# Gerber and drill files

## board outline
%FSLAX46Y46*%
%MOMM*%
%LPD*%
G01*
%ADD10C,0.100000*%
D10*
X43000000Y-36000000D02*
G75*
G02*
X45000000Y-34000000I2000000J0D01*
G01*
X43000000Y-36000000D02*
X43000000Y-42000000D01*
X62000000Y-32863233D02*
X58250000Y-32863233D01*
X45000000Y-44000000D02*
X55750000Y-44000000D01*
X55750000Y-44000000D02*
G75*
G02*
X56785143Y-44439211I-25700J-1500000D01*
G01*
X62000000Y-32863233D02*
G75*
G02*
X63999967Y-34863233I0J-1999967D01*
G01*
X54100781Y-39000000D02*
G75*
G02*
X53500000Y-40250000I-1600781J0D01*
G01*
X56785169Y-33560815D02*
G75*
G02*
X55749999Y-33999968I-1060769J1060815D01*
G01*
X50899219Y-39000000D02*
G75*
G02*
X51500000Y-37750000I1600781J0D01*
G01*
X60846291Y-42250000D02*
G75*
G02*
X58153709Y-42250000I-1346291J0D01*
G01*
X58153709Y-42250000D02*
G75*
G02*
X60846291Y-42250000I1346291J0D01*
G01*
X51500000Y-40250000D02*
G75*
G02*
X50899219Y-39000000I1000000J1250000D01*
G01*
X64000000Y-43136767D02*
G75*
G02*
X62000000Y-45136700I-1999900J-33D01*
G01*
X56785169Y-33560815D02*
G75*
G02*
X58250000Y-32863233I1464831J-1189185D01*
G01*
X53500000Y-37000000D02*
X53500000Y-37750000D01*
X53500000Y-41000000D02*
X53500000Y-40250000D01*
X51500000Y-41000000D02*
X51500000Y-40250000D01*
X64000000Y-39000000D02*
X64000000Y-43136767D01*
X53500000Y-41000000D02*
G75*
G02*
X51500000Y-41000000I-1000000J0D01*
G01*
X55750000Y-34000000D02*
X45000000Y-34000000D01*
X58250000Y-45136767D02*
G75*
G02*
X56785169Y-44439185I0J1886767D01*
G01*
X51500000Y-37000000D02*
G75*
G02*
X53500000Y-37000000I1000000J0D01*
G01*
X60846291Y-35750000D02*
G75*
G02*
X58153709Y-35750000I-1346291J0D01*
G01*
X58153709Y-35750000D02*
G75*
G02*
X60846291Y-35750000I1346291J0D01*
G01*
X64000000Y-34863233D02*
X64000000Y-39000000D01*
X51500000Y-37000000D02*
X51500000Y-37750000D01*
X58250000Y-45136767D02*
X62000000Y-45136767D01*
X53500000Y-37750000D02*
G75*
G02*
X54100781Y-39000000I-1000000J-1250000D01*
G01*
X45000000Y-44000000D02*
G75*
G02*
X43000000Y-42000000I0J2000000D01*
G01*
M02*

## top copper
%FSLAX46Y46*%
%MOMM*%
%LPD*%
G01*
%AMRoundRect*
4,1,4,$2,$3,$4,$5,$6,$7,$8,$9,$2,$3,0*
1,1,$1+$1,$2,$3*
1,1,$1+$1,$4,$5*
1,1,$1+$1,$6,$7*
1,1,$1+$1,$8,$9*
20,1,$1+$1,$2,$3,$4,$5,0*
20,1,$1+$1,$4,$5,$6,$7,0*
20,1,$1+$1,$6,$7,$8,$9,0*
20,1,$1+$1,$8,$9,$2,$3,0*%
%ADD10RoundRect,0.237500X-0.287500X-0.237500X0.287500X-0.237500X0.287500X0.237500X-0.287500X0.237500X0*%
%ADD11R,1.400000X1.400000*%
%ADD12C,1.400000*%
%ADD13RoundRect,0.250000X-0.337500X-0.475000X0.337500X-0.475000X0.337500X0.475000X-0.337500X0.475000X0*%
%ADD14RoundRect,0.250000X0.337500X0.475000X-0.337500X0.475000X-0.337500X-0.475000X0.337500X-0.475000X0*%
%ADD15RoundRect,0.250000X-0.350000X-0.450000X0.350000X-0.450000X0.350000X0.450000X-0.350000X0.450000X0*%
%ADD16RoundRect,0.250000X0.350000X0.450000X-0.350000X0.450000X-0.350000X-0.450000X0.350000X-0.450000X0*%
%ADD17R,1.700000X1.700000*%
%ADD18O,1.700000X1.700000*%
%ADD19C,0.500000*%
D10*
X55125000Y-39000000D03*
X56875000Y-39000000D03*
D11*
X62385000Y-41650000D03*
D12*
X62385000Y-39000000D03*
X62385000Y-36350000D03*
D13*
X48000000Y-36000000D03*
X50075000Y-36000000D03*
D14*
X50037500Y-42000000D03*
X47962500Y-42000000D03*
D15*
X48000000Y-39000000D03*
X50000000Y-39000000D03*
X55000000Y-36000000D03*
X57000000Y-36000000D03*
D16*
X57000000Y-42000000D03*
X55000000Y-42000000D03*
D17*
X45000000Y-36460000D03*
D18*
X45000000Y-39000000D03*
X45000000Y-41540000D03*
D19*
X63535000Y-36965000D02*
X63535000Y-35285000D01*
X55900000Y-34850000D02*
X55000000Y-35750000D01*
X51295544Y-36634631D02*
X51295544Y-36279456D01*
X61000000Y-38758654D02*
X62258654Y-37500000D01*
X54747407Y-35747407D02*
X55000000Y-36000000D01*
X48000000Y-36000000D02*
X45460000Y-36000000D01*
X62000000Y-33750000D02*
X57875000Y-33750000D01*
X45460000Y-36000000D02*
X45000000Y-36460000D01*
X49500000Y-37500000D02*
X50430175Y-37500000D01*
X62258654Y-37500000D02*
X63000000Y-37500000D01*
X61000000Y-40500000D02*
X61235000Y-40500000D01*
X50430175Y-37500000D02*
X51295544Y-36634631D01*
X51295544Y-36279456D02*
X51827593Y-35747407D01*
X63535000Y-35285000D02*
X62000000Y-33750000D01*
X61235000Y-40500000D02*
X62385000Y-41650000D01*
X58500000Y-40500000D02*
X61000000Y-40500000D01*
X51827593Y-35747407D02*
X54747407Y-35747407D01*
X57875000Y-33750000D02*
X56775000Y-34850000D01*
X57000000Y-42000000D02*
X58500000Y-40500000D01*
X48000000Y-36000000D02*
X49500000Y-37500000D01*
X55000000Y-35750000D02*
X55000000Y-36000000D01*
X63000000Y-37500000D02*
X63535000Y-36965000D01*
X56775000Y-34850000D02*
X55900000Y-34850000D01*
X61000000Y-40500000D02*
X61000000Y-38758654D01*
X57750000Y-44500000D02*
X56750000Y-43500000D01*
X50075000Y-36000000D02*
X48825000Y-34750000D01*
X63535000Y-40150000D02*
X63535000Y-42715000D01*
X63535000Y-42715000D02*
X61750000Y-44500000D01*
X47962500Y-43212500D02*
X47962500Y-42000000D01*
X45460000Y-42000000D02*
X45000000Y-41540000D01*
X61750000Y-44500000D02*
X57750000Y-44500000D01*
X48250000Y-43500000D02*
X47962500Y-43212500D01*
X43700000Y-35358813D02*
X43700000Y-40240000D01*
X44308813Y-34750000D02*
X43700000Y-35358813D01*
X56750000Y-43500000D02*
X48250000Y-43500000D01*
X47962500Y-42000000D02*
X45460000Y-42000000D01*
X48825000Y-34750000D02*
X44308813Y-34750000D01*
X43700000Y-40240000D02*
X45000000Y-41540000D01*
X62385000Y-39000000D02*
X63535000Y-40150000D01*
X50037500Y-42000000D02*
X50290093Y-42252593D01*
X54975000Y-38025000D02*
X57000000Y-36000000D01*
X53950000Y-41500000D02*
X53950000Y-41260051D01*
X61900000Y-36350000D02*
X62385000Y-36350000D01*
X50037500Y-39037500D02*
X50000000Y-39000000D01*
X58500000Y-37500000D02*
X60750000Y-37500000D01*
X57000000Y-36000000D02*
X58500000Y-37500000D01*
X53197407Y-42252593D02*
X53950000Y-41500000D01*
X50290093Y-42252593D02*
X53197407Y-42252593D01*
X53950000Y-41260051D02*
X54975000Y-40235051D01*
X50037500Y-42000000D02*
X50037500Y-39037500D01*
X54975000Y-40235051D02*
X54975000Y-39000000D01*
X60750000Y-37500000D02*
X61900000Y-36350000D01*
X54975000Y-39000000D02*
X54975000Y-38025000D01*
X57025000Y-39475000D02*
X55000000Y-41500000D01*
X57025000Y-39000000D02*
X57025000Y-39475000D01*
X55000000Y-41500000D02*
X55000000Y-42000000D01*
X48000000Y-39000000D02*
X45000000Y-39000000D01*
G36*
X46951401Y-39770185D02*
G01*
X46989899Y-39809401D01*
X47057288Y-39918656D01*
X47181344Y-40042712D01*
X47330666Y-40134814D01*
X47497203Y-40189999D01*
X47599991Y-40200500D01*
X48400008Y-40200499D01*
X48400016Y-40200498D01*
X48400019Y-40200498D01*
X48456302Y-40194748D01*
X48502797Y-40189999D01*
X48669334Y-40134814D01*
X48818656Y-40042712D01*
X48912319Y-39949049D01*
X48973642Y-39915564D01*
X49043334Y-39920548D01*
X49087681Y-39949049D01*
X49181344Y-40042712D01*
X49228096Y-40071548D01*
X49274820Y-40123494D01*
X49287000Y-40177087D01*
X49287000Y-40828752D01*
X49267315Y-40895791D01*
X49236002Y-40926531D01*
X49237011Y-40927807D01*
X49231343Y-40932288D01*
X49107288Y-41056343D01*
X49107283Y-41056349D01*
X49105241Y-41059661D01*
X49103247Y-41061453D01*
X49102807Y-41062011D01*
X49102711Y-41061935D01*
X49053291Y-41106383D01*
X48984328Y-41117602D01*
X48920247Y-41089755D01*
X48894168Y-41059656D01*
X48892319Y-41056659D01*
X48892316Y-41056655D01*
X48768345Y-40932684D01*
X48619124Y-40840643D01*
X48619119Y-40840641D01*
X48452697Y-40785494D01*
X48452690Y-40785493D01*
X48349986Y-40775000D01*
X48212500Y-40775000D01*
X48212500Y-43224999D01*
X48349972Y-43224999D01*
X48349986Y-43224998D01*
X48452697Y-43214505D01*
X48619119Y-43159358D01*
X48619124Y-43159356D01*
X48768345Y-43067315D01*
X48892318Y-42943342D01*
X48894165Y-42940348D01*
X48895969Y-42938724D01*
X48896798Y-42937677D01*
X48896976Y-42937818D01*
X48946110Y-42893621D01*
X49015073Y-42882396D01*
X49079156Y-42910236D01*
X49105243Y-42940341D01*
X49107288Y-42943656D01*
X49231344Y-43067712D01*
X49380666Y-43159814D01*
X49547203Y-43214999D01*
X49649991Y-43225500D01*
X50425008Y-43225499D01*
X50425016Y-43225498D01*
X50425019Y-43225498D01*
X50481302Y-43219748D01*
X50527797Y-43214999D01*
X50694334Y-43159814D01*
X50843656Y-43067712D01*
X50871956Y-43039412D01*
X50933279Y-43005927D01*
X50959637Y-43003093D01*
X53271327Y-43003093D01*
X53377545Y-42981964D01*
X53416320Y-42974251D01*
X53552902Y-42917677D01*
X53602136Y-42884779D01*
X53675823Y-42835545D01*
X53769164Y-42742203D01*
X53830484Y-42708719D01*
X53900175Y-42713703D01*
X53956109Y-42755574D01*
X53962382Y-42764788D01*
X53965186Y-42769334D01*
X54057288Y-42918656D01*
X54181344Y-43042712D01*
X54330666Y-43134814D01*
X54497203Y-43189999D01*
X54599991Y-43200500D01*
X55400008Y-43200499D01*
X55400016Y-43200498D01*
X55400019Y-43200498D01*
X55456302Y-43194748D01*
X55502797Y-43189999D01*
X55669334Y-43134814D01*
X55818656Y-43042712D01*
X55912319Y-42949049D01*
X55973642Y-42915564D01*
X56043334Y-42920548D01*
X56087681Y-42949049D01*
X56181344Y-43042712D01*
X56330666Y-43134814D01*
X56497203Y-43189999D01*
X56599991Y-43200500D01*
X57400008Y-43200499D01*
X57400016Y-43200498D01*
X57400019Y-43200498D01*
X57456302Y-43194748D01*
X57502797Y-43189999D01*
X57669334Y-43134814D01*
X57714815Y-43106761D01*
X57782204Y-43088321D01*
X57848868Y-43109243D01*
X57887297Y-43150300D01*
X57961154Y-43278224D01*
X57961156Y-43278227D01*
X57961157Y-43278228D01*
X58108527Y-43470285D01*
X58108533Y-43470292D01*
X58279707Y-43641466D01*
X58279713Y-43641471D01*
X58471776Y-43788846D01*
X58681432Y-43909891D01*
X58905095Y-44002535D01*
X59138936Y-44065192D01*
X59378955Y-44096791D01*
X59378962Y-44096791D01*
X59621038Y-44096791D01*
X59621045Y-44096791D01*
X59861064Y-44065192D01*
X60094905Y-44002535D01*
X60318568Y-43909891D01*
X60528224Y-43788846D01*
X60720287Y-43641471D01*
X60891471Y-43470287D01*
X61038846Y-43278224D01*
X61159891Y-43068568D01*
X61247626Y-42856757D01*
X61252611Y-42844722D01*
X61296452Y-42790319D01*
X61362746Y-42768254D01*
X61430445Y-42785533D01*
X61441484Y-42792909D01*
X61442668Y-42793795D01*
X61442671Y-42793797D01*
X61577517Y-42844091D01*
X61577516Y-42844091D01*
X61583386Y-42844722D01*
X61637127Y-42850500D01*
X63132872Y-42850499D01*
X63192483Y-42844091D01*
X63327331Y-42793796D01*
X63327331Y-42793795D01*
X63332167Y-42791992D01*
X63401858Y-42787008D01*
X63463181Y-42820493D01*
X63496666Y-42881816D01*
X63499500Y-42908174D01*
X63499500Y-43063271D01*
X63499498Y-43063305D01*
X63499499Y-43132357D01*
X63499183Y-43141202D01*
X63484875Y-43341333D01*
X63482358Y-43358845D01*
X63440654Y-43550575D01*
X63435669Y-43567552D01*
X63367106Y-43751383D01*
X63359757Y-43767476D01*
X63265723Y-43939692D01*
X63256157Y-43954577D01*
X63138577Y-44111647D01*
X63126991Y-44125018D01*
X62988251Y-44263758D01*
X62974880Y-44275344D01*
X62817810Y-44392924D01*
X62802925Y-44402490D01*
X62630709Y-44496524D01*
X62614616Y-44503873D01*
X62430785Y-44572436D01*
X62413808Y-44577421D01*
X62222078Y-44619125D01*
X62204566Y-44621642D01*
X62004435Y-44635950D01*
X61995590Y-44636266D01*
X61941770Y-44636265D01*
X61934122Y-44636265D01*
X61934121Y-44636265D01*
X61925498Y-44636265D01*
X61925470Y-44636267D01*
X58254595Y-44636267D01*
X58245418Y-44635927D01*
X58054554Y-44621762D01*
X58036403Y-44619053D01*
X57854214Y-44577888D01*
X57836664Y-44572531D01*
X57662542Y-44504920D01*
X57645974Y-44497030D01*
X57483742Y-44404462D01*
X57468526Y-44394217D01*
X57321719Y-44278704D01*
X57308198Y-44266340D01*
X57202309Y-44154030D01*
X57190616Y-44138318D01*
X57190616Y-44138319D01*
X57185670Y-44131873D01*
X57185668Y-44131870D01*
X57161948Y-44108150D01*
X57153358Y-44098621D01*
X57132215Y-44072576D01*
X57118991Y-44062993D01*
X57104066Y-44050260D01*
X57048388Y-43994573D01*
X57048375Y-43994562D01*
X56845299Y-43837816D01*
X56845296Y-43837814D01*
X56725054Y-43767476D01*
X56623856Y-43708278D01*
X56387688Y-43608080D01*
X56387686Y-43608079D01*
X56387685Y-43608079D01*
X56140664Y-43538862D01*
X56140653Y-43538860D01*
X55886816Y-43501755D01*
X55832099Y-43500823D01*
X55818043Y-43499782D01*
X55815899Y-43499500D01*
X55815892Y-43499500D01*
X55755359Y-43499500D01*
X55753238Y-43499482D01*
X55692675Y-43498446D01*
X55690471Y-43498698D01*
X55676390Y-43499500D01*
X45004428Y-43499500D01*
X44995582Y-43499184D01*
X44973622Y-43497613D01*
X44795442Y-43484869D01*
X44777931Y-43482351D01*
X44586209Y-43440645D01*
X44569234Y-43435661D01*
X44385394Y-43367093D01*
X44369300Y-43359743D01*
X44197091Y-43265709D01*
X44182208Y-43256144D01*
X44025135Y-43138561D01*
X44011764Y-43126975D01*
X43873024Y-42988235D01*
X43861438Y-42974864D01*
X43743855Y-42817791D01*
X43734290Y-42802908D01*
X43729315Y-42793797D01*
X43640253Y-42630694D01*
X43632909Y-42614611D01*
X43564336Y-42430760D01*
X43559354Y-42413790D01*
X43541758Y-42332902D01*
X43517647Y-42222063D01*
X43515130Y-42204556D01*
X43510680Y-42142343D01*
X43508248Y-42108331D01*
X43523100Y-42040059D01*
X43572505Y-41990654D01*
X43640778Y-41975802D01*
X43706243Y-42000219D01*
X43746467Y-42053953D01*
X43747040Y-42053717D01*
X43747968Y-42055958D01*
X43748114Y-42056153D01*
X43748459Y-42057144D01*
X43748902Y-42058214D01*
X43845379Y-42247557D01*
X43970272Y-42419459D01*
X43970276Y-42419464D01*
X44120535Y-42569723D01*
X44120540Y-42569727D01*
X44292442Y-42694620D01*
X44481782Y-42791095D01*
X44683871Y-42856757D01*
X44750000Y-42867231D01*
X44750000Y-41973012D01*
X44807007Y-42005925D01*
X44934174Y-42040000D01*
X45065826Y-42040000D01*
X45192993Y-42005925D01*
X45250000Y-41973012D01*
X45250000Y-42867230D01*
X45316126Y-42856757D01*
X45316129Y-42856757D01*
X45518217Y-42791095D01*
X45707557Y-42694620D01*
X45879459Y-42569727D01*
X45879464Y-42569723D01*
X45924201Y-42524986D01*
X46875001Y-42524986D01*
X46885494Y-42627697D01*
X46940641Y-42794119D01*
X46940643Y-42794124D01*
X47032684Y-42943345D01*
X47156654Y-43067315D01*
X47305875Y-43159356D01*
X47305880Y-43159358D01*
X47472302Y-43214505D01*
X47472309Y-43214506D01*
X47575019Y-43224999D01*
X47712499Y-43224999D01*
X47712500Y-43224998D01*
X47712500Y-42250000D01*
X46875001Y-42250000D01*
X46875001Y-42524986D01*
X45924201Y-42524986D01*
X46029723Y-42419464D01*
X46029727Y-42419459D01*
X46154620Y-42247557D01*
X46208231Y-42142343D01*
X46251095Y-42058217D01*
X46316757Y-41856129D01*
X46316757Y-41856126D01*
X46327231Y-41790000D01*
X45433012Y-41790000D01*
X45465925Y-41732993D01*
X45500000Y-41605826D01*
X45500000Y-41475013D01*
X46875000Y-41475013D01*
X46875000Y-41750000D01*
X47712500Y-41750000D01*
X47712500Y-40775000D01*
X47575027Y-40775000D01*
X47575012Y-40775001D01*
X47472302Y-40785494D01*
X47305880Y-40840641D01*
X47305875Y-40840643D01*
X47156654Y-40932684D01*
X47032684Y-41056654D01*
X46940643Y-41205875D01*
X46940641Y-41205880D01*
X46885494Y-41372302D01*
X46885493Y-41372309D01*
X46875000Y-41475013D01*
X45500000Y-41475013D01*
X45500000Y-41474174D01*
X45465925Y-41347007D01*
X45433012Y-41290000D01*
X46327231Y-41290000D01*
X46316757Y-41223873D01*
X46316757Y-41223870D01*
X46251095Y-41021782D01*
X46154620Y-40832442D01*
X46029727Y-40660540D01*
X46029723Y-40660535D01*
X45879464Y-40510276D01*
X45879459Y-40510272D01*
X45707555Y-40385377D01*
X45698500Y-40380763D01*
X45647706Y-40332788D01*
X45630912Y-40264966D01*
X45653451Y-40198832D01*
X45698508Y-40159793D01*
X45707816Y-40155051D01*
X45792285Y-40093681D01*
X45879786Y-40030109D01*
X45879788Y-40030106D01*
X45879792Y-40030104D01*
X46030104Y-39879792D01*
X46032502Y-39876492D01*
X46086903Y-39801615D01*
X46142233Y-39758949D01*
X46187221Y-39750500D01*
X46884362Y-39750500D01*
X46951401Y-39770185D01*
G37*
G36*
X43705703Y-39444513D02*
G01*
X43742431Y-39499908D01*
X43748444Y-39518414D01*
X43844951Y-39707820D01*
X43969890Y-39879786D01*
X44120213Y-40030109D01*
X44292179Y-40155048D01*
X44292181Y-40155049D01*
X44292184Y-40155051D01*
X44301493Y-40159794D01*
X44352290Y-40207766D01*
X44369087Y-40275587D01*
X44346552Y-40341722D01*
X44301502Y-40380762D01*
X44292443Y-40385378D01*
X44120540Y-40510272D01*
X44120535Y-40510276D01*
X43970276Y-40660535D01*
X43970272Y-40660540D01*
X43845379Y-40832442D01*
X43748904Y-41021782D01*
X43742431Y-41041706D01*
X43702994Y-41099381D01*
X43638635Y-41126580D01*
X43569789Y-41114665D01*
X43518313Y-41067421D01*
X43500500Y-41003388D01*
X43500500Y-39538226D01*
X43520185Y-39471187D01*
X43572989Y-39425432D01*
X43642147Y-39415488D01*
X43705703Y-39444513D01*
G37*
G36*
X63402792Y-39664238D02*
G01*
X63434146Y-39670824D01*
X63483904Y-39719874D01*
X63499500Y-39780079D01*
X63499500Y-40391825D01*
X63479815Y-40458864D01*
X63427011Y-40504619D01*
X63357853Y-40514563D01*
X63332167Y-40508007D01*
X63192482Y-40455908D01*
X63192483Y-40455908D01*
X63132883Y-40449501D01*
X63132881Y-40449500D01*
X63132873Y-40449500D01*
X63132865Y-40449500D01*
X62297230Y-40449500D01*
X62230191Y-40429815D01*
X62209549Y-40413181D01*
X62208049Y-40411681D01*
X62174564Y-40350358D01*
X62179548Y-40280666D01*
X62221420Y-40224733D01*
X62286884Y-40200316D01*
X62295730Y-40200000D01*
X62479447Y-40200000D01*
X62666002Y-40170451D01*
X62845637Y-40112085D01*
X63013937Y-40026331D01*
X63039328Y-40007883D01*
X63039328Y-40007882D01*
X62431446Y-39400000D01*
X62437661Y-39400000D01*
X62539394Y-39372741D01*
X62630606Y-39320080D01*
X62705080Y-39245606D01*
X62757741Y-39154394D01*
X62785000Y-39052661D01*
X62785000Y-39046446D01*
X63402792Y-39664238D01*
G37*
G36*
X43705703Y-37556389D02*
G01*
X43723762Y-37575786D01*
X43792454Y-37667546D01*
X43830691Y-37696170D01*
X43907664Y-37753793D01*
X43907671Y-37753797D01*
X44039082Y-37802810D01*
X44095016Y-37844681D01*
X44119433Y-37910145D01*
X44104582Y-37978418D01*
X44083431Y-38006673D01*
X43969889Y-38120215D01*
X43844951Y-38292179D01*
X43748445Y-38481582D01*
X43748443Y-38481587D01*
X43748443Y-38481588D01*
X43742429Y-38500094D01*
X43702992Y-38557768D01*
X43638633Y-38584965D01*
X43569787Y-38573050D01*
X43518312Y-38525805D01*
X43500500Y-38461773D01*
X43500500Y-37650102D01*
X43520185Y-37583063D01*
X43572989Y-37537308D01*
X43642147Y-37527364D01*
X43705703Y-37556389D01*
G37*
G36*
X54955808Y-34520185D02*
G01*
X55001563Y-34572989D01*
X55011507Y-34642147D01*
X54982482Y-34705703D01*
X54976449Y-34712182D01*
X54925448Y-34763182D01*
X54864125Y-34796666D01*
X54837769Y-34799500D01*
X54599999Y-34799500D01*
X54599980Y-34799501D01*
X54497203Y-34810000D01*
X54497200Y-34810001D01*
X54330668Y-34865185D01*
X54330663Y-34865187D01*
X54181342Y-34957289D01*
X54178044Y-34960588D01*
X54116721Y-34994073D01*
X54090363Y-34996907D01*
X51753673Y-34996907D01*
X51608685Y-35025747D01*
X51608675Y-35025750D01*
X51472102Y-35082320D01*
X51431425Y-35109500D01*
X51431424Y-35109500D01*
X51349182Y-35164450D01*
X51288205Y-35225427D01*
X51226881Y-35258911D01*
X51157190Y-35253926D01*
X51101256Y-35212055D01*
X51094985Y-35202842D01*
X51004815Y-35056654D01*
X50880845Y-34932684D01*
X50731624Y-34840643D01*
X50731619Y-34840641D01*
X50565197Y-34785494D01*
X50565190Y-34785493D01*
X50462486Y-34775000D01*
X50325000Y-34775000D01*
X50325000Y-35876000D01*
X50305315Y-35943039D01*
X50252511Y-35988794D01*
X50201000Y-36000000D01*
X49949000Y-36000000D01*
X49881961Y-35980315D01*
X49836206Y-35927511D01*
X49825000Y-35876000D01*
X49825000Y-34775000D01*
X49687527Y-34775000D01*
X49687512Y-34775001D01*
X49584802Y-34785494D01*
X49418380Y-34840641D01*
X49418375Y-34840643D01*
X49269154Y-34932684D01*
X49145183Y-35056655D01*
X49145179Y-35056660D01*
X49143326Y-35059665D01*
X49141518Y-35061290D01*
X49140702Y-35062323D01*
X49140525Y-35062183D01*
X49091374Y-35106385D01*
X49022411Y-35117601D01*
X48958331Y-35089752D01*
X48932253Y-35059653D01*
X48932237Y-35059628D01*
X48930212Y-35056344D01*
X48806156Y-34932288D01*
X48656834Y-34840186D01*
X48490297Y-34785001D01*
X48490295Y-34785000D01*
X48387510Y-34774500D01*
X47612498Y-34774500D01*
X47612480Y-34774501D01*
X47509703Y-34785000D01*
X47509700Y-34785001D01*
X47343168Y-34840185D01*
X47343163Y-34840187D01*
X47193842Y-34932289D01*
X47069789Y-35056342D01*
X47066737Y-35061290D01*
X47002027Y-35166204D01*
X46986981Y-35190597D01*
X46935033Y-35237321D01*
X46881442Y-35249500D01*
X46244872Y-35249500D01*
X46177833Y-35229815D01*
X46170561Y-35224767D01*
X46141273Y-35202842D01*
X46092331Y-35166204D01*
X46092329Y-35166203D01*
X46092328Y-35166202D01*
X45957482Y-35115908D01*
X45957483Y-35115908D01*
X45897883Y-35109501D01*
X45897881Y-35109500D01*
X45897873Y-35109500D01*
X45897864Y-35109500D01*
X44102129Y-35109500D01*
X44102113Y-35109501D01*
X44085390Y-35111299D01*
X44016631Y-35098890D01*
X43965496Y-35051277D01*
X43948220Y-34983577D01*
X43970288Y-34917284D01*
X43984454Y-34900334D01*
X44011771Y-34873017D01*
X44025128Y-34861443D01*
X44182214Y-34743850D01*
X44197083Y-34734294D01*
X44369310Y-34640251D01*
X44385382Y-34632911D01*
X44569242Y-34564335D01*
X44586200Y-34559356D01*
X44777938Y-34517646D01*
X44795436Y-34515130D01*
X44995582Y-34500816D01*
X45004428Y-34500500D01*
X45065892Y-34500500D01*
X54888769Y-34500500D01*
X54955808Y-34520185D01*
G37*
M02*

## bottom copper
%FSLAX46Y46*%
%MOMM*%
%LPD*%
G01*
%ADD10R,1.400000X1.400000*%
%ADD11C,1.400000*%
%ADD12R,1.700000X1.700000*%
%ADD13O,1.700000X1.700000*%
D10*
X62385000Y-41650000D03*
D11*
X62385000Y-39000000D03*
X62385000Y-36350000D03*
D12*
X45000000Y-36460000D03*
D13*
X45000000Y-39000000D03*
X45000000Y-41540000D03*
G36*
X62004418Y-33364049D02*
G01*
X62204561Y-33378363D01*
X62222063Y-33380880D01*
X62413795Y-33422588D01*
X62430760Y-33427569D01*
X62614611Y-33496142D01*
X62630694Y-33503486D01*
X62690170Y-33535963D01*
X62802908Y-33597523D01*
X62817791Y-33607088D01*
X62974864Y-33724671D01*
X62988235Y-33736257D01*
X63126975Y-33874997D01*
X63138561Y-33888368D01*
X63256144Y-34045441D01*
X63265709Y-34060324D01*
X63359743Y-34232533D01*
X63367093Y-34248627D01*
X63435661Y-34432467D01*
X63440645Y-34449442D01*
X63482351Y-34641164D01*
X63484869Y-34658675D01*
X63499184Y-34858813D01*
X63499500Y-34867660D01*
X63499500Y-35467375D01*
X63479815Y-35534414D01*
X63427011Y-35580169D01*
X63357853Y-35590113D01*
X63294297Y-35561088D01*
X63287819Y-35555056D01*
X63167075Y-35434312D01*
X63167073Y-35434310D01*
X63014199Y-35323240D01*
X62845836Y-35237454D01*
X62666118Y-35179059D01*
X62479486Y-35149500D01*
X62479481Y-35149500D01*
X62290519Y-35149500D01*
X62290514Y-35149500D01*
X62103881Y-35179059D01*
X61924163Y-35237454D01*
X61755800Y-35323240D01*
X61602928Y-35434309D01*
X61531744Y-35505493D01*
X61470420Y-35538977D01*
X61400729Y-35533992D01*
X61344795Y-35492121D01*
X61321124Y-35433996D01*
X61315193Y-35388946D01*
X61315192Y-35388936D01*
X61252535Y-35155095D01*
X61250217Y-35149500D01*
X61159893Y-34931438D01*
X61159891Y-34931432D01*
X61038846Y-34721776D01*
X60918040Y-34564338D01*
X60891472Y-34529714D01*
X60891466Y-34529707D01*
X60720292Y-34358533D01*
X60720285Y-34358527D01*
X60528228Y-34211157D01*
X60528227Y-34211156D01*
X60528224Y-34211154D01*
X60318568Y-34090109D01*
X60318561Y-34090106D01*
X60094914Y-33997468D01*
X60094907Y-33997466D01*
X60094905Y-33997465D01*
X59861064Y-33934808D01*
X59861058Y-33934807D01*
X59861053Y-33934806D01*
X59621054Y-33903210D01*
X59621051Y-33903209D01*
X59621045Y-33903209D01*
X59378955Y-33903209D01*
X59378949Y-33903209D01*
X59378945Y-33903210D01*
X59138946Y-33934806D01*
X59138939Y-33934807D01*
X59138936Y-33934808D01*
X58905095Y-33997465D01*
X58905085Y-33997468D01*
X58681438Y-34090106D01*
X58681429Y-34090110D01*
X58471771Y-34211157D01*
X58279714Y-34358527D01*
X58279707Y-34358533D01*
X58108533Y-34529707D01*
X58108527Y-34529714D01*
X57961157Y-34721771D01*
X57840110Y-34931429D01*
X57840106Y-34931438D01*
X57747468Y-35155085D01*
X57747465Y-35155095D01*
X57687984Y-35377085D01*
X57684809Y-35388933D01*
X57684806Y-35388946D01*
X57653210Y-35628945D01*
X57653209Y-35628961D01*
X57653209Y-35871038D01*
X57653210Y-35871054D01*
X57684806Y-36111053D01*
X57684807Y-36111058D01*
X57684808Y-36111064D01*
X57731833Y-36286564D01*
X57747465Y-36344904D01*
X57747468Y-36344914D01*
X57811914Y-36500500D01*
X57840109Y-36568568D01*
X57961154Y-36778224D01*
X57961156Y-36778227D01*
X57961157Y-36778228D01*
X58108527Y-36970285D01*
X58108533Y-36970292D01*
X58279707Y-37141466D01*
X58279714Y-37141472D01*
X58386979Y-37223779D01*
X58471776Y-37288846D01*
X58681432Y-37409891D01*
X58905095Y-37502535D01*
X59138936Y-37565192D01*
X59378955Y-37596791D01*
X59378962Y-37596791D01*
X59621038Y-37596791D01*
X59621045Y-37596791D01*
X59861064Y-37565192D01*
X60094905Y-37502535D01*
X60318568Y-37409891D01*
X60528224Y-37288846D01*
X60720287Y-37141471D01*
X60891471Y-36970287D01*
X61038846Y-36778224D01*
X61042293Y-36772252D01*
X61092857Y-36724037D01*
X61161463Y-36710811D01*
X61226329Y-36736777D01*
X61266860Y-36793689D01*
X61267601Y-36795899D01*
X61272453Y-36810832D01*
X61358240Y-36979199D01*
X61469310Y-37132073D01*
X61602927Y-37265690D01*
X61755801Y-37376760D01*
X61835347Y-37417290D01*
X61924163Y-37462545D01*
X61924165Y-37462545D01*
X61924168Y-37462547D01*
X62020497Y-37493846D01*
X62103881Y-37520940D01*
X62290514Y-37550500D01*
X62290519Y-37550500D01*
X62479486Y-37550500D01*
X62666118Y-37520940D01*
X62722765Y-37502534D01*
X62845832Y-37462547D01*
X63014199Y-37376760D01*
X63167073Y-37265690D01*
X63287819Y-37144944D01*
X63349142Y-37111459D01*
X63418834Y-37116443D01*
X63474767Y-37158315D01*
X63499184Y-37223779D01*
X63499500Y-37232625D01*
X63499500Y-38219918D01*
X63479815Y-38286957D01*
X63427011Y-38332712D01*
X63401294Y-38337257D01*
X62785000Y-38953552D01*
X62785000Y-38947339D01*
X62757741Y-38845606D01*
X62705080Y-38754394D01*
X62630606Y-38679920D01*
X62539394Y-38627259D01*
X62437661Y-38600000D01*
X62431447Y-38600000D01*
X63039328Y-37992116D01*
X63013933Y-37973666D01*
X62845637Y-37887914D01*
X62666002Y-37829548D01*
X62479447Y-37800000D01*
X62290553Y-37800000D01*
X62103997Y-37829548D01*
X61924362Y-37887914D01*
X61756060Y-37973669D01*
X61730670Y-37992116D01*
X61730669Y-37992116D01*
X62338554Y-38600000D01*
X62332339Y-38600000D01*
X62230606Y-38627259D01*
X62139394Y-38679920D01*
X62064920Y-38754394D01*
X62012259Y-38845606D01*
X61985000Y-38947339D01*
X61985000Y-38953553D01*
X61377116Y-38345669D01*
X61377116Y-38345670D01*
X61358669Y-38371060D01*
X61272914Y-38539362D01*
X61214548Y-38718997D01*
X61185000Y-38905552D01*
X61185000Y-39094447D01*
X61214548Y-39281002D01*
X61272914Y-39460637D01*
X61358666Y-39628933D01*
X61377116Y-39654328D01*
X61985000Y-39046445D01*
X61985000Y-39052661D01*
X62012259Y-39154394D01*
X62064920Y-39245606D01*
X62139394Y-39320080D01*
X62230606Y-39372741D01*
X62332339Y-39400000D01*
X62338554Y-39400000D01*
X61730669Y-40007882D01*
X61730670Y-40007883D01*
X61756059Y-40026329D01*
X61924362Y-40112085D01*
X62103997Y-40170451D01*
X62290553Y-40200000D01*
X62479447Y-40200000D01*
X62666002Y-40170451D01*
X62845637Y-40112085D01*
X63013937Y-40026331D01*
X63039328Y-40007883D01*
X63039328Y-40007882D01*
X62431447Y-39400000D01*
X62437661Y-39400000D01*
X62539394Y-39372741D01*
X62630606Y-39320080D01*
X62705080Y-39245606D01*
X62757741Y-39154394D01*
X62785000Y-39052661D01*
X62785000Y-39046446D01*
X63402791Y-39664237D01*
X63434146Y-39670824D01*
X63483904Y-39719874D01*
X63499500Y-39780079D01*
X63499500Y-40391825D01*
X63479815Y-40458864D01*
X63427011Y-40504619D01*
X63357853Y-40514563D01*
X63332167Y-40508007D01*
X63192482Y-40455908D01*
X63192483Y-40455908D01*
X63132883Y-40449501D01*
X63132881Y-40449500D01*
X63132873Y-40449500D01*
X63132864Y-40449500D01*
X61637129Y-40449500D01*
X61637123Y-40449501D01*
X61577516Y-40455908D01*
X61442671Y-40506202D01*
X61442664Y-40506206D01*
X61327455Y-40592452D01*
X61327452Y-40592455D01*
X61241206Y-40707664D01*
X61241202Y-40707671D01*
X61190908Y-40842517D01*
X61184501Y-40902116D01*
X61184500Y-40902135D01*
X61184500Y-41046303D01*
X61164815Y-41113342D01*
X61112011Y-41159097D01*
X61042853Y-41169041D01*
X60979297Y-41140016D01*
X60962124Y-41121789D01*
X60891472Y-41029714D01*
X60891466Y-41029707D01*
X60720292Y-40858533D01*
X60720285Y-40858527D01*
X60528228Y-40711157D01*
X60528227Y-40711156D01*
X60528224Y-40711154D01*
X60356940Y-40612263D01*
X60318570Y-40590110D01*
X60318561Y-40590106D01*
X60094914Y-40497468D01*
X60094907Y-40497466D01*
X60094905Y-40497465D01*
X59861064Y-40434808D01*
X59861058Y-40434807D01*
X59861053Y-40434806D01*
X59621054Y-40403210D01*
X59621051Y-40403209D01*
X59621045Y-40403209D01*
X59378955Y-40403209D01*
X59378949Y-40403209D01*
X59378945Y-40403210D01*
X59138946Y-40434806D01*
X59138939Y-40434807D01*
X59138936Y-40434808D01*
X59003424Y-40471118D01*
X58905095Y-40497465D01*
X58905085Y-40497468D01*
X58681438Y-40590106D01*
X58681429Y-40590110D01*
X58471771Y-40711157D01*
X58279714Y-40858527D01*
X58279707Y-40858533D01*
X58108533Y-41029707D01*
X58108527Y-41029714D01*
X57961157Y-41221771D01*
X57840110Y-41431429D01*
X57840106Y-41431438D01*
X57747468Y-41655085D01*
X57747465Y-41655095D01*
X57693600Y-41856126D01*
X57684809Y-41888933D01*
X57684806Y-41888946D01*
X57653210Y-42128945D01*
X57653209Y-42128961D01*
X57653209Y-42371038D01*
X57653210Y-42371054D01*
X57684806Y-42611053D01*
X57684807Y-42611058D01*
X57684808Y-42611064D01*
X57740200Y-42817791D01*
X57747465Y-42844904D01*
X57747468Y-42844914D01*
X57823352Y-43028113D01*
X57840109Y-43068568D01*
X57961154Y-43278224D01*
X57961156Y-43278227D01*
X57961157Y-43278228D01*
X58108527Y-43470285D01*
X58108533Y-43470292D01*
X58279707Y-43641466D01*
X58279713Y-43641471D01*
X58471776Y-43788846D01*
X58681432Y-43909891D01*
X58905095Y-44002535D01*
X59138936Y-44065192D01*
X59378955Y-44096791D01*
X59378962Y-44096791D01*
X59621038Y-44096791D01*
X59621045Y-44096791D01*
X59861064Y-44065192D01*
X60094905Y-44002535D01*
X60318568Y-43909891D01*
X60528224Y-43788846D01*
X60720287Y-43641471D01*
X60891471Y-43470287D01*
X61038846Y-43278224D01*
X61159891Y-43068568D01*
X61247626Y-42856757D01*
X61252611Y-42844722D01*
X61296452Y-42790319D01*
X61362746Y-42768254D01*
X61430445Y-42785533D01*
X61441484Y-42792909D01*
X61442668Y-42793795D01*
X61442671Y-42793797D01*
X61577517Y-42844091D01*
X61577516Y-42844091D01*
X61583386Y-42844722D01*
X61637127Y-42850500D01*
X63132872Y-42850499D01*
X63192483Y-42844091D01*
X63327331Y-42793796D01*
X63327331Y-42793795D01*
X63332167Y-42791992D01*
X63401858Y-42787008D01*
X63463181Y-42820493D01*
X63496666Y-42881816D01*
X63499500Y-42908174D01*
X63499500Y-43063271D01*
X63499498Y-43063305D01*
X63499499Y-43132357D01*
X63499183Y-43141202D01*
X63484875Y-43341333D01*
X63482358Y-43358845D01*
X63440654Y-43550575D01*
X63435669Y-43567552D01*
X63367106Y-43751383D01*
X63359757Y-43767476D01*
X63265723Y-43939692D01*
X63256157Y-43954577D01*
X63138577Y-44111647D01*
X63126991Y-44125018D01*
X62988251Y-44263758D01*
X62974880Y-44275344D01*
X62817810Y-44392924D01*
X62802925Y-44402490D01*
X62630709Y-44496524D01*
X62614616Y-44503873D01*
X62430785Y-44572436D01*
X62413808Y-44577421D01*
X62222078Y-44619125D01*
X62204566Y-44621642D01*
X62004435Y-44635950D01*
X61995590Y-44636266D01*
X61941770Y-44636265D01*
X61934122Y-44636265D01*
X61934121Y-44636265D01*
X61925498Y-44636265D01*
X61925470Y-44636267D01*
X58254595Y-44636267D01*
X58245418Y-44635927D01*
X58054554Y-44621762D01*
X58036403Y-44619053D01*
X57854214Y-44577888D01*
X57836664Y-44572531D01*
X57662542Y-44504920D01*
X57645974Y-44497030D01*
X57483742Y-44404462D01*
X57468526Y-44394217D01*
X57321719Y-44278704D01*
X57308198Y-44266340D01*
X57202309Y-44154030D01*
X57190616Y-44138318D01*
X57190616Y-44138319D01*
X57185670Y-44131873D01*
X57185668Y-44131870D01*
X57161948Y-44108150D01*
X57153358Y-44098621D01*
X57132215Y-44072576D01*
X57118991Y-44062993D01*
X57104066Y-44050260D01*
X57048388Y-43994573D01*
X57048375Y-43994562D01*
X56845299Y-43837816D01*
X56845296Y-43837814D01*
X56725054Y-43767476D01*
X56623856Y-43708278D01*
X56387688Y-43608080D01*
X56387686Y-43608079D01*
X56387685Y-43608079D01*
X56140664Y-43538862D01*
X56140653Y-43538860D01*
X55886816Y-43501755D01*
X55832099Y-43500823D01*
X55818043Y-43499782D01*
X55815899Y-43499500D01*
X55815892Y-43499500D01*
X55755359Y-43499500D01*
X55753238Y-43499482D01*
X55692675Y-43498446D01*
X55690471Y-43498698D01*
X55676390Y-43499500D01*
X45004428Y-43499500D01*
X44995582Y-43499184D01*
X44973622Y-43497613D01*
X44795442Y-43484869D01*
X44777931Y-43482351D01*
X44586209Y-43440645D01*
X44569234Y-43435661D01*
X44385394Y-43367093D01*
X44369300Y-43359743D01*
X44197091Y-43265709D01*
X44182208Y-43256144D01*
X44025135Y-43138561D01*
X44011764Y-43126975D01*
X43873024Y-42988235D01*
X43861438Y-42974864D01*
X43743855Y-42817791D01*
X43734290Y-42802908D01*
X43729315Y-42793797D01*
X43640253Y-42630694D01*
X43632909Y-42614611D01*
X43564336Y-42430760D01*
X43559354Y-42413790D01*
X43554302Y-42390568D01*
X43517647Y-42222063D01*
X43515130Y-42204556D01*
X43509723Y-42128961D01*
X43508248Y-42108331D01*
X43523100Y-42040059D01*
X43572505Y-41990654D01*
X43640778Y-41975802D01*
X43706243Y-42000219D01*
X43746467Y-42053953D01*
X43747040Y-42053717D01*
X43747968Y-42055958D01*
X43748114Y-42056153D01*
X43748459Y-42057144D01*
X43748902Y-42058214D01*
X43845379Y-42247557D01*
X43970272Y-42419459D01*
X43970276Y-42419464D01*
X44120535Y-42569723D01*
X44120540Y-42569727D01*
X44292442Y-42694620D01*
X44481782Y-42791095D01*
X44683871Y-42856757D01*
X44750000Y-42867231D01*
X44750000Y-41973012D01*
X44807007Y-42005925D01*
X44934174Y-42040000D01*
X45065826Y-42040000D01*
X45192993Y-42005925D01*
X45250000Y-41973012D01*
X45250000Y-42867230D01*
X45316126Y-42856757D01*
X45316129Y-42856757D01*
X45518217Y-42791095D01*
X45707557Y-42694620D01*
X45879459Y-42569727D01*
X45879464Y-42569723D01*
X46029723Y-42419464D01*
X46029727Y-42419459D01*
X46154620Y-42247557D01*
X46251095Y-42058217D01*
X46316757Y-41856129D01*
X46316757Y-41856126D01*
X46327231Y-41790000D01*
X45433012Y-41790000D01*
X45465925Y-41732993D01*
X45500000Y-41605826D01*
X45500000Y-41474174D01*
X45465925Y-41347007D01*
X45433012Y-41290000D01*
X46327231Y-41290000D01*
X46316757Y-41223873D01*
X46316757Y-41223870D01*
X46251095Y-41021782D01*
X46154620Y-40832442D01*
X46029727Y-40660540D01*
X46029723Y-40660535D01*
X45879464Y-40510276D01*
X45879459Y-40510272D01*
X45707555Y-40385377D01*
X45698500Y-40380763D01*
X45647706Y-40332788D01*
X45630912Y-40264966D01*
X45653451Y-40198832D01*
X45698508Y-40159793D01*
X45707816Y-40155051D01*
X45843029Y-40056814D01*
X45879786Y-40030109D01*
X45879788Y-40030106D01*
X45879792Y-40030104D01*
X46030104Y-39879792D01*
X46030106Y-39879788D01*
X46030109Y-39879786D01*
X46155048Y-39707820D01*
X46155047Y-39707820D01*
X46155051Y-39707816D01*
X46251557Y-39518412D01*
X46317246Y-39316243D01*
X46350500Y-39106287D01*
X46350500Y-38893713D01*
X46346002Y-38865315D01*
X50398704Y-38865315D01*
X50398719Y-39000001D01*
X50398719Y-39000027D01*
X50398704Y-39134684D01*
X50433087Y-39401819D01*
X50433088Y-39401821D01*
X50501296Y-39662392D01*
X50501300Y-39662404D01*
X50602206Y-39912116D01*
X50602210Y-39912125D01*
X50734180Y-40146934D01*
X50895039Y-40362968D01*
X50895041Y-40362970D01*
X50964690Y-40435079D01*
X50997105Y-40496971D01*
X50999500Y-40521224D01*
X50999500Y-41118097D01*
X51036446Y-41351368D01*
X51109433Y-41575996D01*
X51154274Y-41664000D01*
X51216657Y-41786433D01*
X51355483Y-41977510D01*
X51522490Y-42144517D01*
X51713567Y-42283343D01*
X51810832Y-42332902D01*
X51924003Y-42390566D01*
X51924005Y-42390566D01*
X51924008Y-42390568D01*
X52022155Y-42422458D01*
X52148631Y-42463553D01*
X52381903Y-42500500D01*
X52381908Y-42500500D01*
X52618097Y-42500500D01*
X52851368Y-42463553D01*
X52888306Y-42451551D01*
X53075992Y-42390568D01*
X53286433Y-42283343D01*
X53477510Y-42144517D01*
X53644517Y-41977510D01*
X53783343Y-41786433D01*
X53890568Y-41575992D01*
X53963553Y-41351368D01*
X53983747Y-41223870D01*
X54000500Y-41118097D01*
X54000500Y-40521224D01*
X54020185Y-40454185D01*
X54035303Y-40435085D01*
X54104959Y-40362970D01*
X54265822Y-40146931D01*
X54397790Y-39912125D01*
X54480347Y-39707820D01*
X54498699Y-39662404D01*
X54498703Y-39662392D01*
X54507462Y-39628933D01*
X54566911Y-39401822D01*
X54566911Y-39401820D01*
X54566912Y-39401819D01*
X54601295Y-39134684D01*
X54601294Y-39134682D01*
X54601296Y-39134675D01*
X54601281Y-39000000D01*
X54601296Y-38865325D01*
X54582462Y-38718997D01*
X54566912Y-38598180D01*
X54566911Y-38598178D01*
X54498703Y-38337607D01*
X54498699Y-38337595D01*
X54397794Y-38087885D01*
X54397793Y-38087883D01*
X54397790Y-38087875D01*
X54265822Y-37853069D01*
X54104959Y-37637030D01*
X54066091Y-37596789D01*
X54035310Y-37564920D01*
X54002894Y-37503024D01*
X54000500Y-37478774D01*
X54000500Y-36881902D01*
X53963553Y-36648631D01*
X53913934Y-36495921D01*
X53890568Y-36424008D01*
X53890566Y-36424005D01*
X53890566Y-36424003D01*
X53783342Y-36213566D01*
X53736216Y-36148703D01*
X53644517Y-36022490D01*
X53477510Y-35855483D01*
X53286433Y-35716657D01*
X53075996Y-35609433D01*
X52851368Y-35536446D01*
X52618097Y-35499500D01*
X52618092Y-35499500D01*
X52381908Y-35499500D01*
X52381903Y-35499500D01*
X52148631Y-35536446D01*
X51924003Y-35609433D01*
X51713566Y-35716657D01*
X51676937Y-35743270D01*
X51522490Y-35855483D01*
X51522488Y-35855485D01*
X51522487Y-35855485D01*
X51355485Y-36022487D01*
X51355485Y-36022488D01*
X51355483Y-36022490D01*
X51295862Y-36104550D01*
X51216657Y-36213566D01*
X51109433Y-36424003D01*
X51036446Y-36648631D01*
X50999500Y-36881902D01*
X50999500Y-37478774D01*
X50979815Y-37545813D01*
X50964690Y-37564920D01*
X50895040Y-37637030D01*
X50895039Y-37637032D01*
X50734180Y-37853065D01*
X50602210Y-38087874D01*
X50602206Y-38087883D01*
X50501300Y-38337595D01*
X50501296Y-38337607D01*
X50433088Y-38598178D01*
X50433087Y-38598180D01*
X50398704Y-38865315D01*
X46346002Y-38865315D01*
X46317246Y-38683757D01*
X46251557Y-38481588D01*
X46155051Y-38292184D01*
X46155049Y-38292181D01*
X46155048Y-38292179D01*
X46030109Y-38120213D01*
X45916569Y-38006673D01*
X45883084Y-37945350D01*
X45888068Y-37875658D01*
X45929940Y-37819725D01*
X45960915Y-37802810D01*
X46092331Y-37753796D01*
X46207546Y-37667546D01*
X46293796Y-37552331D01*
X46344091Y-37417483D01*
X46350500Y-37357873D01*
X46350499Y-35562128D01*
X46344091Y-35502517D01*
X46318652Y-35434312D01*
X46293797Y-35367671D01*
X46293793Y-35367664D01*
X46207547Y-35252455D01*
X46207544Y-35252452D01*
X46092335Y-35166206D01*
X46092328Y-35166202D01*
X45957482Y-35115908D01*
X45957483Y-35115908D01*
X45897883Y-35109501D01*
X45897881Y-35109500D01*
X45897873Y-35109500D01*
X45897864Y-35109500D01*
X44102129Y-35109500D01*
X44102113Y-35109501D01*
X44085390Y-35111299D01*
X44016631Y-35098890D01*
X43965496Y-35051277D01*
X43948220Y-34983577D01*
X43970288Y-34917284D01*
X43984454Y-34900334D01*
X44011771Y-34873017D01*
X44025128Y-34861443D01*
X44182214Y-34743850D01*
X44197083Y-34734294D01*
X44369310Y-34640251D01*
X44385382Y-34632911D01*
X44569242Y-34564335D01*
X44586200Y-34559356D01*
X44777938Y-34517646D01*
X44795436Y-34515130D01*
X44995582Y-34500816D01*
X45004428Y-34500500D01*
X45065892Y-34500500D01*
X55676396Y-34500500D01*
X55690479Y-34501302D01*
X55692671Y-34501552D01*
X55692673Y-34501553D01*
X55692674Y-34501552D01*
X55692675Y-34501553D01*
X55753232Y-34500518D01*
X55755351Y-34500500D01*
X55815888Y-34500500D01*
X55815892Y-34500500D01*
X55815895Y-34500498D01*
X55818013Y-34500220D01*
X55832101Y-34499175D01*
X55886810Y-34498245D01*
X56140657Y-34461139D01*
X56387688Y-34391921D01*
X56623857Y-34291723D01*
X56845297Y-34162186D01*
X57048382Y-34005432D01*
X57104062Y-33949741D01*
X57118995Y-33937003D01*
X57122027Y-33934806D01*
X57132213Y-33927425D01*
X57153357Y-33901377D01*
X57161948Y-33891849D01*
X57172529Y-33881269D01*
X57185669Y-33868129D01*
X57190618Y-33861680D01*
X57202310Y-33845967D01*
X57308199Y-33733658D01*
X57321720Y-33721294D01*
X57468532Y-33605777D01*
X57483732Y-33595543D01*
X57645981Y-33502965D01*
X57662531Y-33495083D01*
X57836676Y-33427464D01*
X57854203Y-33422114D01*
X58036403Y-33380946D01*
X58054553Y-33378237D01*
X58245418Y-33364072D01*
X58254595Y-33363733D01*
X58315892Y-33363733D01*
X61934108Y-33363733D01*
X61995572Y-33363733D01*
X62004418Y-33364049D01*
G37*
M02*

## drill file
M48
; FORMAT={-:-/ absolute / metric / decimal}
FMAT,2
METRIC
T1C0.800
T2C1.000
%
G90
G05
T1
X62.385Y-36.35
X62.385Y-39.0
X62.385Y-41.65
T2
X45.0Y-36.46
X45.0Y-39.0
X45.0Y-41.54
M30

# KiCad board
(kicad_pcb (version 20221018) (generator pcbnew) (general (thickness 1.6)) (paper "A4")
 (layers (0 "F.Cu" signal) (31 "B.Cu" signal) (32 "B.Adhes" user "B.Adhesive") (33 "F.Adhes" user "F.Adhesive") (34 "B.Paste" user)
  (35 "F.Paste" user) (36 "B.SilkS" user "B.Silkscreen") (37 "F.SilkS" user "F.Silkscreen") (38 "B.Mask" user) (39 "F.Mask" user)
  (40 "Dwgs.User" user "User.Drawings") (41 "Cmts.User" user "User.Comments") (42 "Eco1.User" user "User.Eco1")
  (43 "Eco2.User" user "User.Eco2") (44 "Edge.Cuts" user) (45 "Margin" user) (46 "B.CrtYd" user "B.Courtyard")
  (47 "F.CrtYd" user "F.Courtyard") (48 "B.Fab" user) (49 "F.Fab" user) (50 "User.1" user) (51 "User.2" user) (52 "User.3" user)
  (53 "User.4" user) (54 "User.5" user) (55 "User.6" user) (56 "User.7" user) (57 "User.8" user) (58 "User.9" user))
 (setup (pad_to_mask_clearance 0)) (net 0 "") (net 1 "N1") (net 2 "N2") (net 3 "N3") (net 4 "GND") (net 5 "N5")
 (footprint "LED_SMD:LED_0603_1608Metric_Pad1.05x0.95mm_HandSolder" (layer "F.Cu") (at 56 39)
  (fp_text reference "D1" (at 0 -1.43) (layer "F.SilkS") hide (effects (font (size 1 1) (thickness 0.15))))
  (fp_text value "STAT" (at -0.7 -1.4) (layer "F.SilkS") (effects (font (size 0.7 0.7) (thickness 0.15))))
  (pad "1" smd roundrect (at -0.875 0) (size 1.05 0.95) (layers "F.Cu" "F.Paste" "F.Mask") (roundrect_rratio 0.25) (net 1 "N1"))
  (pad "2" smd roundrect (at 0.875 0) (size 1.05 0.95) (layers "F.Cu" "F.Paste" "F.Mask") (roundrect_rratio 0.25) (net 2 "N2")))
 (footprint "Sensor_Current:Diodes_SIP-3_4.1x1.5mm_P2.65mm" (layer "F.Cu") (at 62.385 41.65 90)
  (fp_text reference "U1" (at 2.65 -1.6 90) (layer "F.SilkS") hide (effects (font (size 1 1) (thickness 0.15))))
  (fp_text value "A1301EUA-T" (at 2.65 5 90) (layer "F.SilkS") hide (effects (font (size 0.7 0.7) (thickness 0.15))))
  (pad "1" thru_hole rect (at 0 0 90) (size 1.4 1.4) (drill 0.8) (layers "*.Cu" "*.Mask") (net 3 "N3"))
  (pad "2" thru_hole circle (at 2.65 0 90) (size 1.4 1.4) (drill 0.8) (layers "*.Cu" "*.Mask") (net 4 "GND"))
  (pad "3" thru_hole circle (at 5.3 0 90) (size 1.4 1.4) (drill 0.8) (layers "*.Cu" "*.Mask") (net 1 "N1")))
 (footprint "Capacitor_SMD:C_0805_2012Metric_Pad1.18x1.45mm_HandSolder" (layer "F.Cu") (at 49.0375 36)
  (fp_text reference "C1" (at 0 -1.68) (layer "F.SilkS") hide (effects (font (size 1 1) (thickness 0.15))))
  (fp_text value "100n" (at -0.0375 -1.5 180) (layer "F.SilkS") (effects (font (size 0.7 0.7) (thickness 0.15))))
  (pad "1" smd roundrect (at -1.0375 0) (size 1.175 1.45) (layers "F.Cu" "F.Paste" "F.Mask") (roundrect_rratio 0.212766) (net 3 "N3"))
  (pad "2" smd roundrect (at 1.0375 0) (size 1.175 1.45) (layers "F.Cu" "F.Paste" "F.Mask") (roundrect_rratio 0.212766) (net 4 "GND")))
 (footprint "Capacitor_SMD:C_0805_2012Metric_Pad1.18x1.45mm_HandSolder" (layer "F.Cu") (at 49 42 180)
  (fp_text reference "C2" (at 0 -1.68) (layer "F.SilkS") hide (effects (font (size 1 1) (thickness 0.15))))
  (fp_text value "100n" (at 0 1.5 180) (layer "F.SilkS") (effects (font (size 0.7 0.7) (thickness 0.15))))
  (pad "1" smd roundrect (at -1.0375 0 180) (size 1.175 1.45) (layers "F.Cu" "F.Paste" "F.Mask") (roundrect_rratio 0.212766) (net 1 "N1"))
  (pad "2" smd roundrect (at 1.0375 0 180) (size 1.175 1.45) (layers "F.Cu" "F.Paste" "F.Mask") (roundrect_rratio 0.212766) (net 4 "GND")))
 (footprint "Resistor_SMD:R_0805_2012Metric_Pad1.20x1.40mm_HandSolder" (layer "F.Cu") (at 49 39)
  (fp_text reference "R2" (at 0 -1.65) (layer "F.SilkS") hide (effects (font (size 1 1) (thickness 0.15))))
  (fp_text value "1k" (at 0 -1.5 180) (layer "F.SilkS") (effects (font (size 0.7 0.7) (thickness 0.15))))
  (pad "1" smd roundrect (at -1 0) (size 1.2 1.4) (layers "F.Cu" "F.Paste" "F.Mask") (roundrect_rratio 0.208333) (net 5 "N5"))
  (pad "2" smd roundrect (at 1 0) (size 1.2 1.4) (layers "F.Cu" "F.Paste" "F.Mask") (roundrect_rratio 0.208333) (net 1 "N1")))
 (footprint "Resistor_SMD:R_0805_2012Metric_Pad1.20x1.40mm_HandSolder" (layer "F.Cu") (at 56 36)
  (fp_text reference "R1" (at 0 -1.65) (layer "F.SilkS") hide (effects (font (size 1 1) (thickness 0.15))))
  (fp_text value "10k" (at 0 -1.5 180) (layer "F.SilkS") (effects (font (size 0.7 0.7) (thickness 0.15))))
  (pad "1" smd roundrect (at -1 0) (size 1.2 1.4) (layers "F.Cu" "F.Paste" "F.Mask") (roundrect_rratio 0.208333) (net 3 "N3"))
  (pad "2" smd roundrect (at 1 0) (size 1.2 1.4) (layers "F.Cu" "F.Paste" "F.Mask") (roundrect_rratio 0.208333) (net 1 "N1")))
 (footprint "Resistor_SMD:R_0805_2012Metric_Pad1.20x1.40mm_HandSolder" (layer "F.Cu") (at 56 42 180)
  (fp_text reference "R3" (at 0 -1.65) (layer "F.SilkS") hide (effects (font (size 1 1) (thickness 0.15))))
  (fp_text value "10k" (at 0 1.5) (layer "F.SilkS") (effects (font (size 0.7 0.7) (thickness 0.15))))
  (pad "1" smd roundrect (at -1 0 180) (size 1.2 1.4) (layers "F.Cu" "F.Paste" "F.Mask") (roundrect_rratio 0.208333) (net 3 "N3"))
  (pad "2" smd roundrect (at 1 0 180) (size 1.2 1.4) (layers "F.Cu" "F.Paste" "F.Mask") (roundrect_rratio 0.208333) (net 2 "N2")))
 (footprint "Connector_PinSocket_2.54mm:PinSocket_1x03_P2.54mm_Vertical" (layer "F.Cu") (at 45 36.46)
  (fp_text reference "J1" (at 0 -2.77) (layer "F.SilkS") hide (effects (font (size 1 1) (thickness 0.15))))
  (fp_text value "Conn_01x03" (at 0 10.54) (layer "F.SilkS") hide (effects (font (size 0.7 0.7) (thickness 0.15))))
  (pad "1" thru_hole rect (at 0 0) (size 1.7 1.7) (drill 1) (layers "*.Cu" "*.Mask") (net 3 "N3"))
  (pad "2" thru_hole oval (at 0 2.54) (size 1.7 1.7) (drill 1) (layers "*.Cu" "*.Mask") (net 5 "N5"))
  (pad "3" thru_hole oval (at 0 5.08) (size 1.7 1.7) (drill 1) (layers "*.Cu" "*.Mask") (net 4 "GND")))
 (gr_arc (start 43 36) (mid 43.585786 34.585786) (end 45 34) (stroke (width 0.1) (type default)) (layer "Edge.Cuts"))
 (gr_line (start 43 36) (end 43 42) (stroke (width 0.1) (type default)) (layer "Edge.Cuts"))
 (gr_line (start 62 32.863233) (end 58.25 32.863233) (stroke (width 0.1) (type default)) (layer "Edge.Cuts"))
 (gr_line (start 45 44) (end 55.75 44) (stroke (width 0.1) (type default)) (layer "Edge.Cuts"))
 (gr_arc (start 55.75 44) (mid 56.310289 44.118937) (end 56.785169 44.439185) (stroke (width 0.1) (type default)) (layer "Edge.Cuts"))
 (gr_arc (start 62 32.863233) (mid 63.414214 33.449019) (end 64 34.863233) (stroke (width 0.1) (type default)) (layer "Edge.Cuts"))
 (gr_arc (start 54.100781 39) (mid 53.942789 39.69344) (end 53.5 40.25) (stroke (width 0.1) (type default)) (layer "Edge.Cuts"))
 (gr_arc (start 56.785169 33.560815) (mid 56.310289 33.881064) (end 55.75 34) (stroke (width 0.1) (type default)) (layer "Edge.Cuts"))
 (gr_arc (start 50.899219 39) (mid 51.057211 38.30656) (end 51.5 37.75) (stroke (width 0.1) (type default)) (layer "Edge.Cuts"))
 (gr_circle (center 59.5 42.25) (end 60.75 41.75) (stroke (width 0.1) (type default)) (fill none) (layer "Edge.Cuts"))
 (gr_arc (start 51.5 40.25) (mid 51.057211 39.69344) (end 50.899219 39) (stroke (width 0.1) (type default)) (layer "Edge.Cuts"))
 (gr_arc (start 64 43.136767) (mid 63.414225 44.551002) (end 62 45.136767) (stroke (width 0.1) (type default)) (layer "Edge.Cuts"))
 (gr_arc (start 56.785169 33.560815) (mid 57.438774 33.046532) (end 58.25 32.863233) (stroke (width 0.1) (type default)) (layer "Edge.Cuts"))
 (gr_line (start 53.5 37) (end 53.5 37.75) (stroke (width 0.1) (type default)) (layer "Edge.Cuts"))
 (gr_line (start 53.5 41) (end 53.5 40.25) (stroke (width 0.1) (type default)) (layer "Edge.Cuts"))
 (gr_line (start 51.5 41) (end 51.5 40.25) (stroke (width 0.1) (type default)) (layer "Edge.Cuts"))
 (gr_line (start 64 39) (end 64 43.136767) (stroke (width 0.1) (type default)) (layer "Edge.Cuts"))
 (gr_arc (start 53.5 41) (mid 52.5 42) (end 51.5 41) (stroke (width 0.1) (type default)) (layer "Edge.Cuts"))
 (gr_line (start 55.75 34) (end 45 34) (stroke (width 0.1) (type default)) (layer "Edge.Cuts"))
 (gr_arc (start 58.25 45.136767) (mid 57.438774 44.953468) (end 56.785169 44.439185) (stroke (width 0.1) (type default)) (layer "Edge.Cuts"))
 (gr_arc (start 51.5 37) (mid 52.5 36) (end 53.5 37) (stroke (width 0.1) (type default)) (layer "Edge.Cuts"))
 (gr_circle (center 59.5 35.75) (end 60.75 35.25) (stroke (width 0.1) (type default)) (fill none) (layer "Edge.Cuts"))
 (gr_line (start 64 34.863233) (end 64 39) (stroke (width 0.1) (type default)) (layer "Edge.Cuts"))
 (gr_line (start 51.5 37) (end 51.5 37.75) (stroke (width 0.1) (type default)) (layer "Edge.Cuts"))
 (gr_line (start 58.25 45.136767) (end 62 45.136767) (stroke (width 0.1) (type default)) (layer "Edge.Cuts"))
 (gr_arc (start 53.5 37.75) (mid 53.942789 38.30656) (end 54.100781 39) (stroke (width 0.1) (type default)) (layer "Edge.Cuts"))
 (gr_arc (start 45 44) (mid 43.585786 43.414214) (end 43 42) (stroke (width 0.1) (type default)) (layer "Edge.Cuts"))
 (segment (start 63.535 36.965) (end 63.535 35.285) (width 0.5) (layer "F.Cu") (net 3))
 (segment (start 55.9 34.85) (end 55 35.75) (width 0.5) (layer "F.Cu") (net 3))
 (segment (start 51.295544 36.634631) (end 51.295544 36.279456) (width 0.5) (layer "F.Cu") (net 3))
 (segment (start 61 38.758654) (end 62.258654 37.5) (width 0.5) (layer "F.Cu") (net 3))
 (segment (start 54.747407 35.747407) (end 55 36) (width 0.5) (layer "F.Cu") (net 3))
 (segment (start 48 36) (end 45.46 36) (width 0.5) (layer "F.Cu") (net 3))
 (segment (start 62 33.75) (end 57.875 33.75) (width 0.5) (layer "F.Cu") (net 3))
 (segment (start 45.46 36) (end 45 36.46) (width 0.5) (layer "F.Cu") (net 3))
 (segment (start 49.5 37.5) (end 50.430175 37.5) (width 0.5) (layer "F.Cu") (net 3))
 (segment (start 62.258654 37.5) (end 63 37.5) (width 0.5) (layer "F.Cu") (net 3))
 (segment (start 61 40.5) (end 61.235 40.5) (width 0.5) (layer "F.Cu") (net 3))
 (segment (start 50.430175 37.5) (end 51.295544 36.634631) (width 0.5) (layer "F.Cu") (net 3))
 (segment (start 51.295544 36.279456) (end 51.827593 35.747407) (width 0.5) (layer "F.Cu") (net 3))
 (segment (start 63.535 35.285) (end 62 33.75) (width 0.5) (layer "F.Cu") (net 3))
 (segment (start 61.235 40.5) (end 62.385 41.65) (width 0.5) (layer "F.Cu") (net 3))
 (segment (start 58.5 40.5) (end 61 40.5) (width 0.5) (layer "F.Cu") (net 3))
 (segment (start 51.827593 35.747407) (end 54.747407 35.747407) (width 0.5) (layer "F.Cu") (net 3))
 (segment (start 57.875 33.75) (end 56.775 34.85) (width 0.5) (layer "F.Cu") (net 3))
 (segment (start 57 42) (end 58.5 40.5) (width 0.5) (layer "F.Cu") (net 3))
 (segment (start 48 36) (end 49.5 37.5) (width 0.5) (layer "F.Cu") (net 3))
 (segment (start 55 35.75) (end 55 36) (width 0.5) (layer "F.Cu") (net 3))
 (segment (start 63 37.5) (end 63.535 36.965) (width 0.5) (layer "F.Cu") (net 3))
 (segment (start 56.775 34.85) (end 55.9 34.85) (width 0.5) (layer "F.Cu") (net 3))
 (segment (start 61 40.5) (end 61 38.758654) (width 0.5) (layer "F.Cu") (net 3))
 (segment (start 57.75 44.5) (end 56.75 43.5) (width 0.5) (layer "F.Cu") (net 4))
 (segment (start 50.075 36) (end 48.825 34.75) (width 0.5) (layer "F.Cu") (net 4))
 (segment (start 63.535 40.15) (end 63.535 42.715) (width 0.5) (layer "F.Cu") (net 4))
 (segment (start 63.535 42.715) (end 61.75 44.5) (width 0.5) (layer "F.Cu") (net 4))
 (segment (start 47.9625 43.2125) (end 47.9625 42) (width 0.5) (layer "F.Cu") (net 4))
 (segment (start 45.46 42) (end 45 41.54) (width 0.5) (layer "F.Cu") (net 4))
 (segment (start 61.75 44.5) (end 57.75 44.5) (width 0.5) (layer "F.Cu") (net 4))
 (segment (start 48.25 43.5) (end 47.9625 43.2125) (width 0.5) (layer "F.Cu") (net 4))
 (segment (start 43.7 35.358813) (end 43.7 40.24) (width 0.5) (layer "F.Cu") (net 4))
 (segment (start 44.308813 34.75) (end 43.7 35.358813) (width 0.5) (layer "F.Cu") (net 4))
 (segment (start 56.75 43.5) (end 48.25 43.5) (width 0.5) (layer "F.Cu") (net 4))
 (segment (start 47.9625 42) (end 45.46 42) (width 0.5) (layer "F.Cu") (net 4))
 (segment (start 48.825 34.75) (end 44.308813 34.75) (width 0.5) (layer "F.Cu") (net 4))
 (segment (start 43.7 40.24) (end 45 41.54) (width 0.5) (layer "F.Cu") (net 4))
 (segment (start 62.385 39) (end 63.535 40.15) (width 0.5) (layer "F.Cu") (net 4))
 (segment (start 50.0375 42) (end 50.290093 42.252593) (width 0.5) (layer "F.Cu") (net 1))
 (segment (start 54.975 38.025) (end 57 36) (width 0.5) (layer "F.Cu") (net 1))
 (segment (start 53.95 41.5) (end 53.95 41.260051) (width 0.5) (layer "F.Cu") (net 1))
 (segment (start 61.9 36.35) (end 62.385 36.35) (width 0.5) (layer "F.Cu") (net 1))
 (segment (start 50.0375 39.0375) (end 50 39) (width 0.5) (layer "F.Cu") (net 1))
 (segment (start 58.5 37.5) (end 60.75 37.5) (width 0.5) (layer "F.Cu") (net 1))
 (segment (start 57 36) (end 58.5 37.5) (width 0.5) (layer "F.Cu") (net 1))
 (segment (start 53.197407 42.252593) (end 53.95 41.5) (width 0.5) (layer "F.Cu") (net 1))
 (segment (start 50.290093 42.252593) (end 53.197407 42.252593) (width 0.5) (layer "F.Cu") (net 1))
 (segment (start 53.95 41.260051) (end 54.975 40.235051) (width 0.5) (layer "F.Cu") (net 1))
 (segment (start 50.0375 42) (end 50.0375 39.0375) (width 0.5) (layer "F.Cu") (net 1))
 (segment (start 54.975 40.235051) (end 54.975 39) (width 0.5) (layer "F.Cu") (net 1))
 (segment (start 60.75 37.5) (end 61.9 36.35) (width 0.5) (layer "F.Cu") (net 1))
 (segment (start 54.975 39) (end 54.975 38.025) (width 0.5) (layer "F.Cu") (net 1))
 (segment (start 57.025 39.475) (end 55 41.5) (width 0.5) (layer "F.Cu") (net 2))
 (segment (start 57.025 39) (end 57.025 39.475) (width 0.5) (layer "F.Cu") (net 2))
 (segment (start 55 41.5) (end 55 42) (width 0.5) (layer "F.Cu") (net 2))
 (segment (start 48 39) (end 45 39) (width 0.5) (layer "F.Cu") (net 5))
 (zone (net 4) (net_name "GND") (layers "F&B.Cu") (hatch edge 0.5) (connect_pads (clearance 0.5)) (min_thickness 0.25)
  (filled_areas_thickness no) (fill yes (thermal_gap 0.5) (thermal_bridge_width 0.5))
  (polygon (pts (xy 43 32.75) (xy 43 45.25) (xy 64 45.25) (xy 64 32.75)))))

